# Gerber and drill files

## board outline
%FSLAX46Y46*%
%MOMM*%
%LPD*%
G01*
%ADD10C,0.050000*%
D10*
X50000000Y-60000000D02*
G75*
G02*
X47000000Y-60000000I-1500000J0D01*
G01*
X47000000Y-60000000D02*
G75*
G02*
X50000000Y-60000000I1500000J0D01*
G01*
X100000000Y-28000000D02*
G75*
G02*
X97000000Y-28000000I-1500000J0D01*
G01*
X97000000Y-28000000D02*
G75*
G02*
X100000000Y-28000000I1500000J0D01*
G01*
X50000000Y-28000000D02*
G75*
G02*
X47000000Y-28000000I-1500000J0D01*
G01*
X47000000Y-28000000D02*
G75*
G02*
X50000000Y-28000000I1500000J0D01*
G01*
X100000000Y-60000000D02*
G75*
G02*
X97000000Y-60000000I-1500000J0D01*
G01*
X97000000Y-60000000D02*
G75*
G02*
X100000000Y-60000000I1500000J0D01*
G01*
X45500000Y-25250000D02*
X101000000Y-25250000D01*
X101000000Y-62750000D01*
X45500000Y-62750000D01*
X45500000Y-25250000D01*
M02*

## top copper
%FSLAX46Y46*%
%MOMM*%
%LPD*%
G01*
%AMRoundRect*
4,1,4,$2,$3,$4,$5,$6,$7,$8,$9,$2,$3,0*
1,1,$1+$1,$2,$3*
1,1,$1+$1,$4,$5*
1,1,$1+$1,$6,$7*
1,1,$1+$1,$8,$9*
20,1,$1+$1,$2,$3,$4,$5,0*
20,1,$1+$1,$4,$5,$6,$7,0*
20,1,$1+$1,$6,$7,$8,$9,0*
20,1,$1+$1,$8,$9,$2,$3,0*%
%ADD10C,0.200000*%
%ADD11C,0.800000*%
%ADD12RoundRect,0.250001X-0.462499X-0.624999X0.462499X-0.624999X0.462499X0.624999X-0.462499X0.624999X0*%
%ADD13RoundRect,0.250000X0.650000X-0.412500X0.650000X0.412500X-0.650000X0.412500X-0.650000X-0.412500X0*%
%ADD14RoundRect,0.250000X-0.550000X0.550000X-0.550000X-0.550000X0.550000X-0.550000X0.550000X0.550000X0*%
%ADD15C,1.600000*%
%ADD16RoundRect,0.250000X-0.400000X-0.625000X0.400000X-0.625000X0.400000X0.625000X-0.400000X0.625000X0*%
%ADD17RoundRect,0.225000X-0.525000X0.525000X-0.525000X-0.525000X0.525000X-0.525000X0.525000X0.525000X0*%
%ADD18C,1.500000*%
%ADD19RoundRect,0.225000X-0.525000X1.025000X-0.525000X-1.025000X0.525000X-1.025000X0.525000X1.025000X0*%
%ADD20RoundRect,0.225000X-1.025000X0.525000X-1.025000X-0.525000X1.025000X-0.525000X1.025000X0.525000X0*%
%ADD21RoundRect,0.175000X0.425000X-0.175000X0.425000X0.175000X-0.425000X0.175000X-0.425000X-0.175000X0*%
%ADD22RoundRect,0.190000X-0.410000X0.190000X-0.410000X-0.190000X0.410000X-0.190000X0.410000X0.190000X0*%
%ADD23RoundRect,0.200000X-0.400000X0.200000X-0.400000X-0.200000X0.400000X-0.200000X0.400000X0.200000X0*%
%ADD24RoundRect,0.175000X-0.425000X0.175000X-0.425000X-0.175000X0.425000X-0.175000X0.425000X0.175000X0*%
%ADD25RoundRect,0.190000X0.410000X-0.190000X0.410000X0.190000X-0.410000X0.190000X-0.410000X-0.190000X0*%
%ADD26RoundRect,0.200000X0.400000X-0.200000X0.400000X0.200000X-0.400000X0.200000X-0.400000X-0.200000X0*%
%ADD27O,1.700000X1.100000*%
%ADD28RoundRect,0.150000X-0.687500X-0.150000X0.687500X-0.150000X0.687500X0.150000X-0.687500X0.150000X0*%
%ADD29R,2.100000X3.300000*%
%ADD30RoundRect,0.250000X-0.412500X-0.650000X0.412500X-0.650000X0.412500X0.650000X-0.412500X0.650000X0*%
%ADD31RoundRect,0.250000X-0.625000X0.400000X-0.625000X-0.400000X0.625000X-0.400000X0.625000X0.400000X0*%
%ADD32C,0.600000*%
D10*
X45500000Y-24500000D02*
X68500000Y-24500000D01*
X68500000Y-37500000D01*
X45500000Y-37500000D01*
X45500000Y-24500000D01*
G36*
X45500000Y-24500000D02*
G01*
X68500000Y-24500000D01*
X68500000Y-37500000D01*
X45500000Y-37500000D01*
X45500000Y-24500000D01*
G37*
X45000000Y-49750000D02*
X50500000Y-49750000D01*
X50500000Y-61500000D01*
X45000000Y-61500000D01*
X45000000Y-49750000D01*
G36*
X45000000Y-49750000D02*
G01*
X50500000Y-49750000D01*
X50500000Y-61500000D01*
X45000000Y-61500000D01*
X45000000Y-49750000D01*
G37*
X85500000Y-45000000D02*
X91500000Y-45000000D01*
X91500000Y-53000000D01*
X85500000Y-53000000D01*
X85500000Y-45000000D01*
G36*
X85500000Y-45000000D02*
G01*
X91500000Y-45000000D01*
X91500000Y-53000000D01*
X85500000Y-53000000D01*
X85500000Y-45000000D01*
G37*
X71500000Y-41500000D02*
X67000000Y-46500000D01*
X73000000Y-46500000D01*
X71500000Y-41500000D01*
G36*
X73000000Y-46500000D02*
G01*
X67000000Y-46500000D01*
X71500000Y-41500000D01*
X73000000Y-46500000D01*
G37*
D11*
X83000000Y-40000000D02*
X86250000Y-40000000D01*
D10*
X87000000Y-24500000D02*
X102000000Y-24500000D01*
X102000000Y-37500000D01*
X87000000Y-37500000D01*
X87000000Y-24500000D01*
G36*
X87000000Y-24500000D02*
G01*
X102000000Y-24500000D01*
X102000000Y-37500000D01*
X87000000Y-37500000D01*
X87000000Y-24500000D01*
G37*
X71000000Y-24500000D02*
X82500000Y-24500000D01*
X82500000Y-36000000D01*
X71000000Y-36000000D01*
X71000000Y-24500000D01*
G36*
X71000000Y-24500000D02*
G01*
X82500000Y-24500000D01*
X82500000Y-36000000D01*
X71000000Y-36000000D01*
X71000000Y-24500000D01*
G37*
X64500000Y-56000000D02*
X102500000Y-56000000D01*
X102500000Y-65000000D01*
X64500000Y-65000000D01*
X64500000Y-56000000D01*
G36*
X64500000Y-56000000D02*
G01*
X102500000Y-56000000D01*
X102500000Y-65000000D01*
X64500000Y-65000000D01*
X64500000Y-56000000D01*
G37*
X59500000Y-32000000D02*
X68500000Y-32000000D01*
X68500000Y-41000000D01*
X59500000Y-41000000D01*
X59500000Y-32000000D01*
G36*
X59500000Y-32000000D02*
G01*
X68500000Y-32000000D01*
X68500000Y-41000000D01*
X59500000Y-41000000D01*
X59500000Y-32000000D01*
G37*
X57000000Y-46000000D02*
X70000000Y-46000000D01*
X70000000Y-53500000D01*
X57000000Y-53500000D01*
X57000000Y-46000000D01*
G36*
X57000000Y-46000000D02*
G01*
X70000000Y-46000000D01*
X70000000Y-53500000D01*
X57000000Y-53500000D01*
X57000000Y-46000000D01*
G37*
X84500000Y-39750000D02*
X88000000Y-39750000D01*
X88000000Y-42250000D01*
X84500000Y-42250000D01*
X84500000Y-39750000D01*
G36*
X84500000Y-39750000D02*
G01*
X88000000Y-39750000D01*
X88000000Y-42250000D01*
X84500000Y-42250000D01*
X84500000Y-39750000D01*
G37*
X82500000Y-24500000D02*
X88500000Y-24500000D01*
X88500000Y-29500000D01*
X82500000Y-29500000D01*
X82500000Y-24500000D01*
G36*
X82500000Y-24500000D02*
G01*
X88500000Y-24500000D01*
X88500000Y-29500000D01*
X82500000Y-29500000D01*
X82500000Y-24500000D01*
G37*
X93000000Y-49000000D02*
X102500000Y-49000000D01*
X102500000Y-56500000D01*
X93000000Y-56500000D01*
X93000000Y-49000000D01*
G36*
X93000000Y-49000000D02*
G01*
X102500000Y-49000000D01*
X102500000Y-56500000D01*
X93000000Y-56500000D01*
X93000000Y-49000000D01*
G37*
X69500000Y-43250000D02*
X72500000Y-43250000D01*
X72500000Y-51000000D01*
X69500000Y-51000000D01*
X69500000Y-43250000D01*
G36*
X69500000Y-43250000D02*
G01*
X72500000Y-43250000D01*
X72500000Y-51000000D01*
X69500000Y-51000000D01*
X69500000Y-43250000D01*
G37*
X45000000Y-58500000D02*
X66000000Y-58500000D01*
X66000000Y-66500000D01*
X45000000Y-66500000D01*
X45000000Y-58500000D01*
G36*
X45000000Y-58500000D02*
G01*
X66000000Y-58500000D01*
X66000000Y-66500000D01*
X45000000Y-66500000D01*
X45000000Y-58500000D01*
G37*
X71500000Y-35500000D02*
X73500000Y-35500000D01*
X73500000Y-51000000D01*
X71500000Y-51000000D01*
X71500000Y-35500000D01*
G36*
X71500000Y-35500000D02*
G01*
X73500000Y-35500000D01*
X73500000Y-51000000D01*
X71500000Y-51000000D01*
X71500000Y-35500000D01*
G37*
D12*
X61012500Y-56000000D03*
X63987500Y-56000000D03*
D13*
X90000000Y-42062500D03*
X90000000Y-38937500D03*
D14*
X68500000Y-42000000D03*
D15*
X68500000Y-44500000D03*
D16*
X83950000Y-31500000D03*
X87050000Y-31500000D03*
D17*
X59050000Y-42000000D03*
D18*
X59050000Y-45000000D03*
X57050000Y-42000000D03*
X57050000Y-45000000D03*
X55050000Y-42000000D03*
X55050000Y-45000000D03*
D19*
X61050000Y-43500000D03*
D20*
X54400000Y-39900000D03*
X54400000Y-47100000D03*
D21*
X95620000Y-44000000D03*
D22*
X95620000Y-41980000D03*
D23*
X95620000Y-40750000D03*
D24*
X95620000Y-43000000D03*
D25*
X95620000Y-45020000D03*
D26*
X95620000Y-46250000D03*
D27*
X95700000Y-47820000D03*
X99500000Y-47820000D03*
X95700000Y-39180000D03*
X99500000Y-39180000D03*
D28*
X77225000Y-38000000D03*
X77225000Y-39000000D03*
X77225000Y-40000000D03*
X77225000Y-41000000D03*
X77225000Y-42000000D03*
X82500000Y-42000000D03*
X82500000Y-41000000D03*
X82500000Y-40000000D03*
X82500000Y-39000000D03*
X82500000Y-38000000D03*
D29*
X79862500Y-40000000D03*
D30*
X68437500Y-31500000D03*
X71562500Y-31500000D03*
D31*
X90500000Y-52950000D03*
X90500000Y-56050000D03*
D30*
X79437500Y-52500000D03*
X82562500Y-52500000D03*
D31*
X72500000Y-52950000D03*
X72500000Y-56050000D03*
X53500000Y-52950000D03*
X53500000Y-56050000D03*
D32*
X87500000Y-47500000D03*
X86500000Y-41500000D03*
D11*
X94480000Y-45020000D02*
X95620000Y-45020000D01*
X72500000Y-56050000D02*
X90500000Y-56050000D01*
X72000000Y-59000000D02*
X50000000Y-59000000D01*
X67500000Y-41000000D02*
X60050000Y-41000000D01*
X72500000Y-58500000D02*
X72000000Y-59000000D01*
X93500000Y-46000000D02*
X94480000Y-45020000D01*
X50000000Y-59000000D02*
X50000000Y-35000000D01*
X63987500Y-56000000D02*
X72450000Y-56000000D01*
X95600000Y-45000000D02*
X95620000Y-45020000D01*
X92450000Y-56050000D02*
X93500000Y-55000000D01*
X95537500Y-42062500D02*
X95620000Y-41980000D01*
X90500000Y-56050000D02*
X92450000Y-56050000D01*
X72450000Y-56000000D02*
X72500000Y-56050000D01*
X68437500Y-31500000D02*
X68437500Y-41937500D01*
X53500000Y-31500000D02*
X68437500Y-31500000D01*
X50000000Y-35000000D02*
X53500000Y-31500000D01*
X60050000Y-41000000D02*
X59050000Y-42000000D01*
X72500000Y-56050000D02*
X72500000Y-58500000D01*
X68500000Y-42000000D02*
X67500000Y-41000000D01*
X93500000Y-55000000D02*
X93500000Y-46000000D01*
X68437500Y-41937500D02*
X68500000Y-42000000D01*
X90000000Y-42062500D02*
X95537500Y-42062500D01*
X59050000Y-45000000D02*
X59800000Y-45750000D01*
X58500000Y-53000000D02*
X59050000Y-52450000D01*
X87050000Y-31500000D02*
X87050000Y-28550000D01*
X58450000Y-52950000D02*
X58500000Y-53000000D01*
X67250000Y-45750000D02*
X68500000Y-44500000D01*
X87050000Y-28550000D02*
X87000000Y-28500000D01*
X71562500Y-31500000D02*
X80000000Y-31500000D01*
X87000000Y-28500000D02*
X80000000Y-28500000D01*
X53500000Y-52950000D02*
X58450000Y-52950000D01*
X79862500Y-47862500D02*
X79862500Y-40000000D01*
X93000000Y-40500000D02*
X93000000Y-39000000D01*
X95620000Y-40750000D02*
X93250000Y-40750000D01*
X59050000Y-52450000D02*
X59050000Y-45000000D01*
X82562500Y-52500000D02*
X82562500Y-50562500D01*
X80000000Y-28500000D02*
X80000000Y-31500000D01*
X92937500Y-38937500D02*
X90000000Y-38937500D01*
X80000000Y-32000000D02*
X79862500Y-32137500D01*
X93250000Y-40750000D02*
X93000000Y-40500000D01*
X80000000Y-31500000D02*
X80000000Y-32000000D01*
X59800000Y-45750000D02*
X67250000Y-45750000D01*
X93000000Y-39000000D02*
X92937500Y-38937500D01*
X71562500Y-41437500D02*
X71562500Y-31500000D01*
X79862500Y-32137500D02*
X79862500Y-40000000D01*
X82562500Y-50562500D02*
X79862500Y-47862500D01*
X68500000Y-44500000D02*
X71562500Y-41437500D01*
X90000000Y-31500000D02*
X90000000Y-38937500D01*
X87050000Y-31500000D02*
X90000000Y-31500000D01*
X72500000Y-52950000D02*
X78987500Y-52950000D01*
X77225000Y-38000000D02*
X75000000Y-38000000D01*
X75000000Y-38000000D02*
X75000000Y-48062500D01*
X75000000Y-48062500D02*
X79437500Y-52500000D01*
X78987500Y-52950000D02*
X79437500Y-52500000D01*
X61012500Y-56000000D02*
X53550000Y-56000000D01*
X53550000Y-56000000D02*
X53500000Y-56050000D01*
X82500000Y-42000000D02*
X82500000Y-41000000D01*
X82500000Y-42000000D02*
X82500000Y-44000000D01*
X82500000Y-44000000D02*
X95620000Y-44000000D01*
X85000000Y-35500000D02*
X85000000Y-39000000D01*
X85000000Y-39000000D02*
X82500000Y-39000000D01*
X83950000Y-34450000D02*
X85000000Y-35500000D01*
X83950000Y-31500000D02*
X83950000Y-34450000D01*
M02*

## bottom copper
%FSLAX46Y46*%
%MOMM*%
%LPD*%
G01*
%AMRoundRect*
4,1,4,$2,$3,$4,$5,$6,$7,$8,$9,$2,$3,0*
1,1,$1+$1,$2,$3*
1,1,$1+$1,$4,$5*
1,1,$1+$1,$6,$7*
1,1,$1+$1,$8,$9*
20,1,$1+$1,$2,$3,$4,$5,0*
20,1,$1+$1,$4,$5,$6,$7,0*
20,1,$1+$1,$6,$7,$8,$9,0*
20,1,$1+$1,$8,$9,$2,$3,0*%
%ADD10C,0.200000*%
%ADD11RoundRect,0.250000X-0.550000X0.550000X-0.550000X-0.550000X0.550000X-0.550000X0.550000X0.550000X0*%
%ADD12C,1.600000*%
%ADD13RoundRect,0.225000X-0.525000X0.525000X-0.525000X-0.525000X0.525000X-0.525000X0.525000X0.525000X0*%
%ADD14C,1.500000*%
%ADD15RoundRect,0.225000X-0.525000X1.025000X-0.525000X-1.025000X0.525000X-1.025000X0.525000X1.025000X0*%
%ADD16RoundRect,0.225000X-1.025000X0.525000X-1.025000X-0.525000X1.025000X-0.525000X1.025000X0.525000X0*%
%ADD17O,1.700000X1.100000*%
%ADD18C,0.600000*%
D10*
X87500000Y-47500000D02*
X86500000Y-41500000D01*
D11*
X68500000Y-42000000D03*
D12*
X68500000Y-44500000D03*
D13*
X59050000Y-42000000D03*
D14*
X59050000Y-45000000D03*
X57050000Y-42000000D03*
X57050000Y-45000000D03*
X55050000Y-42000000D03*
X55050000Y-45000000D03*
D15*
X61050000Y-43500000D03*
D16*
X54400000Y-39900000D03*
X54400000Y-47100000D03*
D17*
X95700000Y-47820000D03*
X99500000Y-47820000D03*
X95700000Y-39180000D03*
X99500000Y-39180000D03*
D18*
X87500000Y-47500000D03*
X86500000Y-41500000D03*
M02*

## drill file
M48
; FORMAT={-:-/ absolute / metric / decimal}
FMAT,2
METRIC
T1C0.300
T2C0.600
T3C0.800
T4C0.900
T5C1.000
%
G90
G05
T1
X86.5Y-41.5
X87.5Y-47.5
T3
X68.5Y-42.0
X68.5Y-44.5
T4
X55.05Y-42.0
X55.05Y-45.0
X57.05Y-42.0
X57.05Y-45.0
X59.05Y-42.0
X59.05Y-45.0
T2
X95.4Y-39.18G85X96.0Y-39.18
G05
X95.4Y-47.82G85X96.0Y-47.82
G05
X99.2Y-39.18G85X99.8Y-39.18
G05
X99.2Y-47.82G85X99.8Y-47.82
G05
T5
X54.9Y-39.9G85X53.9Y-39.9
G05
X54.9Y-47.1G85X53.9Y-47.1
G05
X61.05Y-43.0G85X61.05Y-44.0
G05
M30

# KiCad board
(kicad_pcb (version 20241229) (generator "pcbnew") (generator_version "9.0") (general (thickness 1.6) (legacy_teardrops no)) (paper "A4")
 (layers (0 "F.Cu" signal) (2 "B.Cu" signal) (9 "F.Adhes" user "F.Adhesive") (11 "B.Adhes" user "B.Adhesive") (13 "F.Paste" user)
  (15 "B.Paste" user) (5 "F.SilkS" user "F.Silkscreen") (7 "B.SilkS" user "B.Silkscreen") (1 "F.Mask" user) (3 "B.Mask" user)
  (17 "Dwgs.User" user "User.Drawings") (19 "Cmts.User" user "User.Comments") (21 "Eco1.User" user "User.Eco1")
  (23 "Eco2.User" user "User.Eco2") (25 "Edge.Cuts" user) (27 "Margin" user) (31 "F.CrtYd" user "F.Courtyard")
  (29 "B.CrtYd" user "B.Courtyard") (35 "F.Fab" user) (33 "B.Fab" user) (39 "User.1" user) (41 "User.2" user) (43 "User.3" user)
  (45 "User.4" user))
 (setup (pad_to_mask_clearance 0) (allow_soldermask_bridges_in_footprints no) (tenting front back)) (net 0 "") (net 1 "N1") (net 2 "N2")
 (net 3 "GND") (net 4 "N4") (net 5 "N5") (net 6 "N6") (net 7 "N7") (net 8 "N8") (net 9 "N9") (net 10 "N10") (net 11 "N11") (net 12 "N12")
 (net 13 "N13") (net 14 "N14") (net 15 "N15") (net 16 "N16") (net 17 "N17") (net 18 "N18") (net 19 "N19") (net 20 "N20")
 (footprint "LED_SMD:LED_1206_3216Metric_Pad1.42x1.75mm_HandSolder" (layer "F.Cu") (at 62.5 56)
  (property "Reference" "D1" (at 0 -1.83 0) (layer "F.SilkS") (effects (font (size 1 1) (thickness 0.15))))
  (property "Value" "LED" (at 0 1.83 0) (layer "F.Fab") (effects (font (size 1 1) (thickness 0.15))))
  (pad "1" smd roundrect (at -1.4875 0) (size 1.425 1.75) (layers "F.Cu" "F.Mask" "F.Paste") (roundrect_rratio 0.175439) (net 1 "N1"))
  (pad "2" smd roundrect (at 1.4875 0) (size 1.425 1.75) (layers "F.Cu" "F.Mask" "F.Paste") (roundrect_rratio 0.175439) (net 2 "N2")))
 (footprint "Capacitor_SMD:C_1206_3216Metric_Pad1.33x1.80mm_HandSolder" (layer "F.Cu") (at 90 40.5 90)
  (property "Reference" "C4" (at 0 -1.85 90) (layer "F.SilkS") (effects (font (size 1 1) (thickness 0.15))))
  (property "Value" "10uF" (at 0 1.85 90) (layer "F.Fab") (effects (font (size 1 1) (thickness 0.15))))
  (pad "1" smd roundrect (at -1.5625 0 90) (size 1.325 1.8) (layers "F.Cu" "F.Mask" "F.Paste") (roundrect_rratio 0.188679) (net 2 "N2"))
  (pad "2" smd roundrect (at 1.5625 0 90) (size 1.325 1.8) (layers "F.Cu" "F.Mask" "F.Paste") (roundrect_rratio 0.188679) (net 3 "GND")))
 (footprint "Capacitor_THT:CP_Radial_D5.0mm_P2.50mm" (layer "F.Cu") (at 68.5 42 -90)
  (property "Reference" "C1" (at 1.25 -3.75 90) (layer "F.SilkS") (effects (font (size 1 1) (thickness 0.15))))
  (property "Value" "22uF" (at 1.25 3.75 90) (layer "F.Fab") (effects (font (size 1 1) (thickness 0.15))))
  (pad "1" thru_hole roundrect (at 0 0 270) (size 1.6 1.6) (drill 0.8) (layers "*.Cu" "*.Mask") (remove_unused_layers no)
   (roundrect_rratio 0.15625) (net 2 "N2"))
  (pad "2" thru_hole circle (at 2.5 0 270) (size 1.6 1.6) (drill 0.8) (layers "*.Cu" "*.Mask") (remove_unused_layers no) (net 3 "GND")))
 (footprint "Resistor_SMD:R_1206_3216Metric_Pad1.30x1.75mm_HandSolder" (layer "F.Cu") (at 85.5 31.5)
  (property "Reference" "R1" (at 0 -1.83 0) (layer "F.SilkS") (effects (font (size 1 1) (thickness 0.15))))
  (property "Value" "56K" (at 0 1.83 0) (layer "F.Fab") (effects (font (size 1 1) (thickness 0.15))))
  (pad "1" smd roundrect (at -1.55 0) (size 1.3 1.75) (layers "F.Cu" "F.Mask" "F.Paste") (roundrect_rratio 0.192308) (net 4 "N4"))
  (pad "2" smd roundrect (at 1.55 0) (size 1.3 1.75) (layers "F.Cu" "F.Mask" "F.Paste") (roundrect_rratio 0.192308) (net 3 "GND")))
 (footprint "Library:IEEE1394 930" (layer "F.Cu") (at 45.5 43.5 -90)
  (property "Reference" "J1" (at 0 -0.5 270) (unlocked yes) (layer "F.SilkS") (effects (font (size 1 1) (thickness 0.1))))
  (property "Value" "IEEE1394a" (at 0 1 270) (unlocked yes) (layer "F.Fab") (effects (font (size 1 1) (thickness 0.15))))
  (pad "1" thru_hole roundrect (at -1.5 -13.55 270) (size 1.5 1.5) (drill 0.9) (layers "*.Cu" "*.Mask") (remove_unused_layers no)
   (roundrect_rratio 0.15) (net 2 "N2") (thermal_bridge_angle 45))
  (pad "2" thru_hole circle (at 1.5 -13.55 270) (size 1.5 1.5) (drill 0.9) (layers "*.Cu" "*.Mask") (remove_unused_layers no) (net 3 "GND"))
  (pad "3" thru_hole circle (at -1.5 -11.55 270) (size 1.5 1.5) (drill 0.9) (layers "*.Cu" "*.Mask") (remove_unused_layers no) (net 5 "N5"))
  (pad "4" thru_hole circle (at 1.5 -11.55 270) (size 1.5 1.5) (drill 0.9) (layers "*.Cu" "*.Mask") (remove_unused_layers no) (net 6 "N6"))
  (pad "5" thru_hole circle (at -1.5 -9.55 270) (size 1.5 1.5) (drill 0.9) (layers "*.Cu" "*.Mask") (remove_unused_layers no) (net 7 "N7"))
  (pad "6" thru_hole circle (at 1.5 -9.55 270) (size 1.5 1.5) (drill 0.9) (layers "*.Cu" "*.Mask") (remove_unused_layers no) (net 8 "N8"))
  (pad "7" thru_hole roundrect (at 0 -15.55 270) (size 2.5 1.5) (drill oval 2 1) (layers "*.Cu" "*.Mask") (remove_unused_layers no)
   (roundrect_rratio 0.15) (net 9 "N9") (thermal_bridge_angle 45))
  (pad "8" thru_hole roundrect (at -3.6 -8.9 270) (size 1.5 2.5) (drill oval 1 2) (layers "*.Cu" "*.Mask") (remove_unused_layers no)
   (roundrect_rratio 0.15) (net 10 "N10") (thermal_bridge_angle 45))
  (pad "9" thru_hole roundrect (at 3.6 -8.9 270) (size 1.5 2.5) (drill oval 1 2) (layers "*.Cu" "*.Mask") (remove_unused_layers no)
   (roundrect_rratio 0.15) (thermal_bridge_angle 45)))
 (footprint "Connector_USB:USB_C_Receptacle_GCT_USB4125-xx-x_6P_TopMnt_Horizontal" (layer "F.Cu") (at 98.7 43.5 90)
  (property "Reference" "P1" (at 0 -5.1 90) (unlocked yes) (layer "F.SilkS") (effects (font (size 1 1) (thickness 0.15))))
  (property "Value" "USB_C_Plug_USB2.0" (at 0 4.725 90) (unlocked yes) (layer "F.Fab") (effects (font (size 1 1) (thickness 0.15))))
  (pad "A5" smd roundrect (at -0.5 -3.08 90) (size 0.7 1.2) (layers "F.Cu" "F.Mask" "F.Paste") (roundrect_rratio 0.25) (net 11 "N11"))
  (pad "A9" smd roundrect (at 1.52 -3.08 270) (size 0.76 1.2) (layers "F.Cu" "F.Mask" "F.Paste") (roundrect_rratio 0.25) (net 2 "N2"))
  (pad "A12" smd roundrect (at 2.75 -3.08 270) (size 0.8 1.2) (layers "F.Cu" "F.Mask" "F.Paste") (roundrect_rratio 0.25) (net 3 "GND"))
  (pad "B5" smd roundrect (at 0.5 -3.08 270) (size 0.7 1.2) (layers "F.Cu" "F.Mask" "F.Paste") (roundrect_rratio 0.25) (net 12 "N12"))
  (pad "B9" smd roundrect (at -1.52 -3.08 90) (size 0.76 1.2) (layers "F.Cu" "F.Mask" "F.Paste") (roundrect_rratio 0.25) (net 2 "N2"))
  (pad "B12" smd roundrect (at -2.75 -3.08 90) (size 0.8 1.2) (layers "F.Cu" "F.Mask" "F.Paste") (roundrect_rratio 0.25) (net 3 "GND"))
  (pad "S1" thru_hole oval (at -4.32 -3 90) (size 1.1 1.7) (drill oval 0.6 1.2) (layers "*.Cu" "*.Mask" "F.Paste") (remove_unused_layers no)
   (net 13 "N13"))
  (pad "S1" thru_hole oval (at -4.32 0.8 90) (size 1.1 1.7) (drill oval 0.6 1.2) (layers "*.Cu" "*.Mask" "F.Paste")
   (remove_unused_layers no) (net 13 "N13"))
  (pad "S1" thru_hole oval (at 4.32 -3 90) (size 1.1 1.7) (drill oval 0.6 1.2) (layers "*.Cu" "*.Mask" "F.Paste") (remove_unused_layers no)
   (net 13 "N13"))
  (pad "S1" thru_hole oval (at 4.32 0.8 90) (size 1.1 1.7) (drill oval 0.6 1.2) (layers "*.Cu" "*.Mask" "F.Paste") (remove_unused_layers no)
   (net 13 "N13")))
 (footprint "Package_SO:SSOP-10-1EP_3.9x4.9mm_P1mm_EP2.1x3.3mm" (layer "F.Cu") (at 79.8625 40)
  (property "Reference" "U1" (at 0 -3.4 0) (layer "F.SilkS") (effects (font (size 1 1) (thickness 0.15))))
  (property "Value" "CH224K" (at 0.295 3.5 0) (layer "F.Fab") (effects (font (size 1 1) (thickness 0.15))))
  (pad "" smd roundrect (at 0 0) (size 1.69 2.66) (layers "F.Paste") (roundrect_rratio 0.147929))
  (pad "1" smd roundrect (at -2.6375 -2) (size 1.675 0.6) (layers "F.Cu" "F.Mask" "F.Paste") (roundrect_rratio 0.25) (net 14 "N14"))
  (pad "2" smd roundrect (at -2.6375 -1) (size 1.675 0.6) (layers "F.Cu" "F.Mask" "F.Paste") (roundrect_rratio 0.25) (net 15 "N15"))
  (pad "3" smd roundrect (at -2.6375 0) (size 1.675 0.6) (layers "F.Cu" "F.Mask" "F.Paste") (roundrect_rratio 0.25) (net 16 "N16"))
  (pad "4" smd roundrect (at -2.6375 1) (size 1.675 0.6) (layers "F.Cu" "F.Mask" "F.Paste") (roundrect_rratio 0.25) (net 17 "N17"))
  (pad "5" smd roundrect (at -2.6375 2) (size 1.675 0.6) (layers "F.Cu" "F.Mask" "F.Paste") (roundrect_rratio 0.25) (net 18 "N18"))
  (pad "6" smd roundrect (at 2.6375 2) (size 1.675 0.6) (layers "F.Cu" "F.Mask" "F.Paste") (roundrect_rratio 0.25) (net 11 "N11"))
  (pad "7" smd roundrect (at 2.6375 1) (size 1.675 0.6) (layers "F.Cu" "F.Mask" "F.Paste") (roundrect_rratio 0.25) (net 11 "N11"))
  (pad "8" smd roundrect (at 2.6375 0) (size 1.675 0.6) (layers "F.Cu" "F.Mask" "F.Paste") (roundrect_rratio 0.25) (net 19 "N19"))
  (pad "9" smd roundrect (at 2.6375 -1) (size 1.675 0.6) (layers "F.Cu" "F.Mask" "F.Paste") (roundrect_rratio 0.25) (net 4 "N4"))
  (pad "10" smd roundrect (at 2.6375 -2) (size 1.675 0.6) (layers "F.Cu" "F.Mask" "F.Paste") (roundrect_rratio 0.25) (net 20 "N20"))
  (pad "11" smd rect (at 0 0) (size 2.1 3.3) (layers "F.Cu" "F.Mask") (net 3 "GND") (zone_connect 2)))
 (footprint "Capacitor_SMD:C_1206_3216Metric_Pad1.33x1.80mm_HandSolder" (layer "F.Cu") (at 70 31.5)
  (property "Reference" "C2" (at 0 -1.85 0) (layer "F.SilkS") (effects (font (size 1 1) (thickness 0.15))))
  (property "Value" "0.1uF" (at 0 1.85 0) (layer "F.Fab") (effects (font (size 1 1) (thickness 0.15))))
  (pad "1" smd roundrect (at -1.5625 0) (size 1.325 1.8) (layers "F.Cu" "F.Mask" "F.Paste") (roundrect_rratio 0.188679) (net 2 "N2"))
  (pad "2" smd roundrect (at 1.5625 0) (size 1.325 1.8) (layers "F.Cu" "F.Mask" "F.Paste") (roundrect_rratio 0.188679) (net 3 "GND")))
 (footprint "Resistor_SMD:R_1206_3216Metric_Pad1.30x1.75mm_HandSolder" (layer "F.Cu") (at 90.5 54.5 -90)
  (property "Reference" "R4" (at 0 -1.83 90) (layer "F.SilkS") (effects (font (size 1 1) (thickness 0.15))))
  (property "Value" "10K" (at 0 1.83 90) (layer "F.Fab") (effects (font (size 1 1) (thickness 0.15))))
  (pad "1" smd roundrect (at -1.55 0 270) (size 1.3 1.75) (layers "F.Cu" "F.Mask" "F.Paste") (roundrect_rratio 0.192308) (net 19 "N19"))
  (pad "2" smd roundrect (at 1.55 0 270) (size 1.3 1.75) (layers "F.Cu" "F.Mask" "F.Paste") (roundrect_rratio 0.192308) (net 2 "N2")))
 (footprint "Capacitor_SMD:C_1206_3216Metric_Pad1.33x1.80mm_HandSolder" (layer "F.Cu") (at 81 52.5)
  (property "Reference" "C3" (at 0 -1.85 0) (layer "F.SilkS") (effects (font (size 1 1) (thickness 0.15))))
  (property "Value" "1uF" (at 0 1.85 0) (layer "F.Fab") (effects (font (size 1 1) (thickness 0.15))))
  (pad "1" smd roundrect (at -1.5625 0) (size 1.325 1.8) (layers "F.Cu" "F.Mask" "F.Paste") (roundrect_rratio 0.188679) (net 14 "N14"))
  (pad "2" smd roundrect (at 1.5625 0) (size 1.325 1.8) (layers "F.Cu" "F.Mask" "F.Paste") (roundrect_rratio 0.188679) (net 3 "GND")))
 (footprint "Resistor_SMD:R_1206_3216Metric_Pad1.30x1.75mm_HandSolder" (layer "F.Cu") (at 72.5 54.5 -90)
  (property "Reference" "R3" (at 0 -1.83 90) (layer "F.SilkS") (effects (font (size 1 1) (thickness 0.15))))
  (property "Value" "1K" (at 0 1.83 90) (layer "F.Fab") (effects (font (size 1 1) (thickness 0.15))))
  (pad "1" smd roundrect (at -1.55 0 270) (size 1.3 1.75) (layers "F.Cu" "F.Mask" "F.Paste") (roundrect_rratio 0.192308) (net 14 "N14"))
  (pad "2" smd roundrect (at 1.55 0 270) (size 1.3 1.75) (layers "F.Cu" "F.Mask" "F.Paste") (roundrect_rratio 0.192308) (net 2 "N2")))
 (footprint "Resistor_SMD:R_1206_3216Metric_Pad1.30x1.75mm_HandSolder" (layer "F.Cu") (at 53.5 54.5 -90)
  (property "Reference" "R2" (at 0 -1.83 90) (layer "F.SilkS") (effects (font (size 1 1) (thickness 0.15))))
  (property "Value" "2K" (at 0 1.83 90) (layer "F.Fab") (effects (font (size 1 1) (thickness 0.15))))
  (pad "1" smd roundrect (at -1.55 0 270) (size 1.3 1.75) (layers "F.Cu" "F.Mask" "F.Paste") (roundrect_rratio 0.192308) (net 3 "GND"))
  (pad "2" smd roundrect (at 1.55 0 270) (size 1.3 1.75) (layers "F.Cu" "F.Mask" "F.Paste") (roundrect_rratio 0.192308) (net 1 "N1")))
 (gr_rect (start 45.5 24.5) (end 68.5 37.5) (stroke (width 0.2) (type solid)) (fill yes) (layer "F.Cu") (net 2))
 (gr_rect (start 45 49.75) (end 50.5 61.5) (stroke (width 0.2) (type solid)) (fill yes) (layer "F.Cu") (net 2))
 (gr_rect (start 85.5 45) (end 91.5 53) (stroke (width 0.2) (type solid)) (fill yes) (layer "F.Cu") (net 19))
 (gr_poly (pts (xy 71.5 41.5) (xy 67 46.5) (xy 73 46.5)) (stroke (width 0.2) (type solid)) (fill yes) (layer "F.Cu") (net 3))
 (gr_line (start 83 40) (end 86.25 40) (stroke (width 0.8) (type solid)) (layer "F.Cu") (net 19))
 (gr_rect (start 87 24.5) (end 102 37.5) (stroke (width 0.2) (type solid)) (fill yes) (layer "F.Cu") (net 3))
 (gr_rect (start 71 24.5) (end 82.5 36) (stroke (width 0.2) (type solid)) (fill yes) (layer "F.Cu") (net 3))
 (gr_rect (start 64.5 56) (end 102.5 65) (stroke (width 0.2) (type solid)) (fill yes) (layer "F.Cu") (net 2))
 (gr_rect (start 59.5 32) (end 68.5 41) (stroke (width 0.2) (type solid)) (fill yes) (layer "F.Cu") (net 2))
 (gr_rect (start 57 46) (end 70 53.5) (stroke (width 0.2) (type solid)) (fill yes) (layer "F.Cu") (net 3))
 (gr_rect (start 84.5 39.75) (end 88 42.25) (stroke (width 0.2) (type solid)) (fill yes) (layer "F.Cu") (net 19))
 (gr_rect (start 82.5 24.5) (end 88.5 29.5) (stroke (width 0.2) (type solid)) (fill yes) (layer "F.Cu") (net 3))
 (gr_rect (start 93 49) (end 102.5 56.5) (stroke (width 0.2) (type solid)) (fill yes) (layer "F.Cu") (net 2))
 (gr_rect (start 69.5 43.25) (end 72.5 51) (stroke (width 0.2) (type solid)) (fill yes) (layer "F.Cu") (net 3))
 (gr_rect (start 45 58.5) (end 66 66.5) (stroke (width 0.2) (type solid)) (fill yes) (layer "F.Cu") (net 2))
 (gr_rect (start 71.5 35.5) (end 73.5 51) (stroke (width 0.2) (type solid)) (fill yes) (layer "F.Cu") (net 3))
 (gr_line (start 87.5 47.5) (end 86.5 41.5) (stroke (width 0.2) (type default)) (layer "B.Cu") (net 19))
 (gr_circle (center 48.5 60) (end 47 60) (stroke (width 0.05) (type default)) (fill no) (layer "Edge.Cuts"))
 (gr_circle (center 98.5 28) (end 100 28) (stroke (width 0.05) (type default)) (fill no) (layer "Edge.Cuts"))
 (gr_circle (center 48.5 28) (end 47 28) (stroke (width 0.05) (type default)) (fill no) (layer "Edge.Cuts"))
 (gr_circle (center 98.5 60) (end 100 60) (stroke (width 0.05) (type default)) (fill no) (layer "Edge.Cuts"))
 (gr_rect (start 45.5 25.25) (end 101 62.75) (stroke (width 0.05) (type default)) (fill no) (layer "Edge.Cuts"))
 (segment (start 94.48 45.02) (end 95.62 45.02) (width 0.8) (layer "F.Cu") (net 2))
 (segment (start 72.5 56.05) (end 90.5 56.05) (width 0.8) (layer "F.Cu") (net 2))
 (segment (start 72 59) (end 50 59) (width 0.8) (layer "F.Cu") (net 2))
 (segment (start 67.5 41) (end 60.05 41) (width 0.8) (layer "F.Cu") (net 2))
 (segment (start 72.5 58.5) (end 72 59) (width 0.8) (layer "F.Cu") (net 2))
 (segment (start 93.5 46) (end 94.48 45.02) (width 0.8) (layer "F.Cu") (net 2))
 (segment (start 50 59) (end 50 35) (width 0.8) (layer "F.Cu") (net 2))
 (segment (start 63.9875 56) (end 72.45 56) (width 0.8) (layer "F.Cu") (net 2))
 (segment (start 95.6 45) (end 95.62 45.02) (width 0.8) (layer "F.Cu") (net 2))
 (segment (start 92.45 56.05) (end 93.5 55) (width 0.8) (layer "F.Cu") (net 2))
 (segment (start 95.5375 42.0625) (end 95.62 41.98) (width 0.8) (layer "F.Cu") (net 2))
 (segment (start 90.5 56.05) (end 92.45 56.05) (width 0.8) (layer "F.Cu") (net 2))
 (segment (start 72.45 56) (end 72.5 56.05) (width 0.8) (layer "F.Cu") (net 2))
 (segment (start 68.4375 31.5) (end 68.4375 41.9375) (width 0.8) (layer "F.Cu") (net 2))
 (segment (start 53.5 31.5) (end 68.4375 31.5) (width 0.8) (layer "F.Cu") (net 2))
 (segment (start 50 35) (end 53.5 31.5) (width 0.8) (layer "F.Cu") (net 2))
 (segment (start 60.05 41) (end 59.05 42) (width 0.8) (layer "F.Cu") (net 2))
 (segment (start 72.5 56.05) (end 72.5 58.5) (width 0.8) (layer "F.Cu") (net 2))
 (segment (start 68.5 42) (end 67.5 41) (width 0.8) (layer "F.Cu") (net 2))
 (segment (start 93.5 55) (end 93.5 46) (width 0.8) (layer "F.Cu") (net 2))
 (segment (start 68.4375 41.9375) (end 68.5 42) (width 0.8) (layer "F.Cu") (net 2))
 (segment (start 90 42.0625) (end 95.5375 42.0625) (width 0.8) (layer "F.Cu") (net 2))
 (segment (start 59.05 45) (end 59.8 45.75) (width 0.8) (layer "F.Cu") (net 3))
 (segment (start 58.5 53) (end 59.05 52.45) (width 0.8) (layer "F.Cu") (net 3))
 (segment (start 87.05 31.5) (end 87.05 28.55) (width 0.8) (layer "F.Cu") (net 3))
 (segment (start 58.45 52.95) (end 58.5 53) (width 0.8) (layer "F.Cu") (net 3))
 (segment (start 67.25 45.75) (end 68.5 44.5) (width 0.8) (layer "F.Cu") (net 3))
 (segment (start 87.05 28.55) (end 87 28.5) (width 0.8) (layer "F.Cu") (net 3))
 (segment (start 71.5625 31.5) (end 80 31.5) (width 0.8) (layer "F.Cu") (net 3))
 (segment (start 87 28.5) (end 80 28.5) (width 0.8) (layer "F.Cu") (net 3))
 (segment (start 53.5 52.95) (end 58.45 52.95) (width 0.8) (layer "F.Cu") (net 3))
 (segment (start 79.8625 47.8625) (end 79.8625 40) (width 0.8) (layer "F.Cu") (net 3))
 (segment (start 93 40.5) (end 93 39) (width 0.8) (layer "F.Cu") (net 3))
 (segment (start 95.62 40.75) (end 93.25 40.75) (width 0.8) (layer "F.Cu") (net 3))
 (segment (start 59.05 52.45) (end 59.05 45) (width 0.8) (layer "F.Cu") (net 3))
 (segment (start 82.5625 52.5) (end 82.5625 50.5625) (width 0.8) (layer "F.Cu") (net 3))
 (segment (start 80 28.5) (end 80 31.5) (width 0.8) (layer "F.Cu") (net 3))
 (segment (start 92.9375 38.9375) (end 90 38.9375) (width 0.8) (layer "F.Cu") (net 3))
 (segment (start 80 32) (end 79.8625 32.1375) (width 0.8) (layer "F.Cu") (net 3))
 (segment (start 93.25 40.75) (end 93 40.5) (width 0.8) (layer "F.Cu") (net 3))
 (segment (start 80 31.5) (end 80 32) (width 0.8) (layer "F.Cu") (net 3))
 (segment (start 59.8 45.75) (end 67.25 45.75) (width 0.8) (layer "F.Cu") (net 3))
 (segment (start 93 39) (end 92.9375 38.9375) (width 0.8) (layer "F.Cu") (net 3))
 (segment (start 71.5625 41.4375) (end 71.5625 31.5) (width 0.8) (layer "F.Cu") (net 3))
 (segment (start 79.8625 32.1375) (end 79.8625 40) (width 0.8) (layer "F.Cu") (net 3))
 (segment (start 82.5625 50.5625) (end 79.8625 47.8625) (width 0.8) (layer "F.Cu") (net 3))
 (segment (start 68.5 44.5) (end 71.5625 41.4375) (width 0.8) (layer "F.Cu") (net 3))
 (segment (start 90 31.5) (end 90 38.9375) (width 0.8) (layer "F.Cu") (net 3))
 (segment (start 87.05 31.5) (end 90 31.5) (width 0.8) (layer "F.Cu") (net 3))
 (segment (start 72.5 52.95) (end 78.9875 52.95) (width 0.8) (layer "F.Cu") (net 14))
 (segment (start 77.225 38) (end 75 38) (width 0.8) (layer "F.Cu") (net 14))
 (segment (start 75 38) (end 75 48.0625) (width 0.8) (layer "F.Cu") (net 14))
 (segment (start 75 48.0625) (end 79.4375 52.5) (width 0.8) (layer "F.Cu") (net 14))
 (segment (start 78.9875 52.95) (end 79.4375 52.5) (width 0.8) (layer "F.Cu") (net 14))
 (segment (start 61.0125 56) (end 53.55 56) (width 0.8) (layer "F.Cu") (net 1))
 (segment (start 53.55 56) (end 53.5 56.05) (width 0.8) (layer "F.Cu") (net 1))
 (segment (start 82.5 42) (end 82.5 41) (width 0.8) (layer "F.Cu") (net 11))
 (segment (start 82.5 42) (end 82.5 44) (width 0.8) (layer "F.Cu") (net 11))
 (segment (start 82.5 44) (end 95.62 44) (width 0.8) (layer "F.Cu") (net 11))
 (segment (start 85 35.5) (end 85 39) (width 0.8) (layer "F.Cu") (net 4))
 (segment (start 85 39) (end 82.5 39) (width 0.8) (layer "F.Cu") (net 4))
 (segment (start 83.95 34.45) (end 85 35.5) (width 0.8) (layer "F.Cu") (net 4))
 (segment (start 83.95 31.5) (end 83.95 34.45) (width 0.8) (layer "F.Cu") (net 4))
 (via (at 87.5 47.5) (size 0.6) (drill 0.3) (layers "F.Cu" "B.Cu") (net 19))
 (via (at 86.5 41.5) (size 0.6) (drill 0.3) (layers "F.Cu" "B.Cu") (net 19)))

